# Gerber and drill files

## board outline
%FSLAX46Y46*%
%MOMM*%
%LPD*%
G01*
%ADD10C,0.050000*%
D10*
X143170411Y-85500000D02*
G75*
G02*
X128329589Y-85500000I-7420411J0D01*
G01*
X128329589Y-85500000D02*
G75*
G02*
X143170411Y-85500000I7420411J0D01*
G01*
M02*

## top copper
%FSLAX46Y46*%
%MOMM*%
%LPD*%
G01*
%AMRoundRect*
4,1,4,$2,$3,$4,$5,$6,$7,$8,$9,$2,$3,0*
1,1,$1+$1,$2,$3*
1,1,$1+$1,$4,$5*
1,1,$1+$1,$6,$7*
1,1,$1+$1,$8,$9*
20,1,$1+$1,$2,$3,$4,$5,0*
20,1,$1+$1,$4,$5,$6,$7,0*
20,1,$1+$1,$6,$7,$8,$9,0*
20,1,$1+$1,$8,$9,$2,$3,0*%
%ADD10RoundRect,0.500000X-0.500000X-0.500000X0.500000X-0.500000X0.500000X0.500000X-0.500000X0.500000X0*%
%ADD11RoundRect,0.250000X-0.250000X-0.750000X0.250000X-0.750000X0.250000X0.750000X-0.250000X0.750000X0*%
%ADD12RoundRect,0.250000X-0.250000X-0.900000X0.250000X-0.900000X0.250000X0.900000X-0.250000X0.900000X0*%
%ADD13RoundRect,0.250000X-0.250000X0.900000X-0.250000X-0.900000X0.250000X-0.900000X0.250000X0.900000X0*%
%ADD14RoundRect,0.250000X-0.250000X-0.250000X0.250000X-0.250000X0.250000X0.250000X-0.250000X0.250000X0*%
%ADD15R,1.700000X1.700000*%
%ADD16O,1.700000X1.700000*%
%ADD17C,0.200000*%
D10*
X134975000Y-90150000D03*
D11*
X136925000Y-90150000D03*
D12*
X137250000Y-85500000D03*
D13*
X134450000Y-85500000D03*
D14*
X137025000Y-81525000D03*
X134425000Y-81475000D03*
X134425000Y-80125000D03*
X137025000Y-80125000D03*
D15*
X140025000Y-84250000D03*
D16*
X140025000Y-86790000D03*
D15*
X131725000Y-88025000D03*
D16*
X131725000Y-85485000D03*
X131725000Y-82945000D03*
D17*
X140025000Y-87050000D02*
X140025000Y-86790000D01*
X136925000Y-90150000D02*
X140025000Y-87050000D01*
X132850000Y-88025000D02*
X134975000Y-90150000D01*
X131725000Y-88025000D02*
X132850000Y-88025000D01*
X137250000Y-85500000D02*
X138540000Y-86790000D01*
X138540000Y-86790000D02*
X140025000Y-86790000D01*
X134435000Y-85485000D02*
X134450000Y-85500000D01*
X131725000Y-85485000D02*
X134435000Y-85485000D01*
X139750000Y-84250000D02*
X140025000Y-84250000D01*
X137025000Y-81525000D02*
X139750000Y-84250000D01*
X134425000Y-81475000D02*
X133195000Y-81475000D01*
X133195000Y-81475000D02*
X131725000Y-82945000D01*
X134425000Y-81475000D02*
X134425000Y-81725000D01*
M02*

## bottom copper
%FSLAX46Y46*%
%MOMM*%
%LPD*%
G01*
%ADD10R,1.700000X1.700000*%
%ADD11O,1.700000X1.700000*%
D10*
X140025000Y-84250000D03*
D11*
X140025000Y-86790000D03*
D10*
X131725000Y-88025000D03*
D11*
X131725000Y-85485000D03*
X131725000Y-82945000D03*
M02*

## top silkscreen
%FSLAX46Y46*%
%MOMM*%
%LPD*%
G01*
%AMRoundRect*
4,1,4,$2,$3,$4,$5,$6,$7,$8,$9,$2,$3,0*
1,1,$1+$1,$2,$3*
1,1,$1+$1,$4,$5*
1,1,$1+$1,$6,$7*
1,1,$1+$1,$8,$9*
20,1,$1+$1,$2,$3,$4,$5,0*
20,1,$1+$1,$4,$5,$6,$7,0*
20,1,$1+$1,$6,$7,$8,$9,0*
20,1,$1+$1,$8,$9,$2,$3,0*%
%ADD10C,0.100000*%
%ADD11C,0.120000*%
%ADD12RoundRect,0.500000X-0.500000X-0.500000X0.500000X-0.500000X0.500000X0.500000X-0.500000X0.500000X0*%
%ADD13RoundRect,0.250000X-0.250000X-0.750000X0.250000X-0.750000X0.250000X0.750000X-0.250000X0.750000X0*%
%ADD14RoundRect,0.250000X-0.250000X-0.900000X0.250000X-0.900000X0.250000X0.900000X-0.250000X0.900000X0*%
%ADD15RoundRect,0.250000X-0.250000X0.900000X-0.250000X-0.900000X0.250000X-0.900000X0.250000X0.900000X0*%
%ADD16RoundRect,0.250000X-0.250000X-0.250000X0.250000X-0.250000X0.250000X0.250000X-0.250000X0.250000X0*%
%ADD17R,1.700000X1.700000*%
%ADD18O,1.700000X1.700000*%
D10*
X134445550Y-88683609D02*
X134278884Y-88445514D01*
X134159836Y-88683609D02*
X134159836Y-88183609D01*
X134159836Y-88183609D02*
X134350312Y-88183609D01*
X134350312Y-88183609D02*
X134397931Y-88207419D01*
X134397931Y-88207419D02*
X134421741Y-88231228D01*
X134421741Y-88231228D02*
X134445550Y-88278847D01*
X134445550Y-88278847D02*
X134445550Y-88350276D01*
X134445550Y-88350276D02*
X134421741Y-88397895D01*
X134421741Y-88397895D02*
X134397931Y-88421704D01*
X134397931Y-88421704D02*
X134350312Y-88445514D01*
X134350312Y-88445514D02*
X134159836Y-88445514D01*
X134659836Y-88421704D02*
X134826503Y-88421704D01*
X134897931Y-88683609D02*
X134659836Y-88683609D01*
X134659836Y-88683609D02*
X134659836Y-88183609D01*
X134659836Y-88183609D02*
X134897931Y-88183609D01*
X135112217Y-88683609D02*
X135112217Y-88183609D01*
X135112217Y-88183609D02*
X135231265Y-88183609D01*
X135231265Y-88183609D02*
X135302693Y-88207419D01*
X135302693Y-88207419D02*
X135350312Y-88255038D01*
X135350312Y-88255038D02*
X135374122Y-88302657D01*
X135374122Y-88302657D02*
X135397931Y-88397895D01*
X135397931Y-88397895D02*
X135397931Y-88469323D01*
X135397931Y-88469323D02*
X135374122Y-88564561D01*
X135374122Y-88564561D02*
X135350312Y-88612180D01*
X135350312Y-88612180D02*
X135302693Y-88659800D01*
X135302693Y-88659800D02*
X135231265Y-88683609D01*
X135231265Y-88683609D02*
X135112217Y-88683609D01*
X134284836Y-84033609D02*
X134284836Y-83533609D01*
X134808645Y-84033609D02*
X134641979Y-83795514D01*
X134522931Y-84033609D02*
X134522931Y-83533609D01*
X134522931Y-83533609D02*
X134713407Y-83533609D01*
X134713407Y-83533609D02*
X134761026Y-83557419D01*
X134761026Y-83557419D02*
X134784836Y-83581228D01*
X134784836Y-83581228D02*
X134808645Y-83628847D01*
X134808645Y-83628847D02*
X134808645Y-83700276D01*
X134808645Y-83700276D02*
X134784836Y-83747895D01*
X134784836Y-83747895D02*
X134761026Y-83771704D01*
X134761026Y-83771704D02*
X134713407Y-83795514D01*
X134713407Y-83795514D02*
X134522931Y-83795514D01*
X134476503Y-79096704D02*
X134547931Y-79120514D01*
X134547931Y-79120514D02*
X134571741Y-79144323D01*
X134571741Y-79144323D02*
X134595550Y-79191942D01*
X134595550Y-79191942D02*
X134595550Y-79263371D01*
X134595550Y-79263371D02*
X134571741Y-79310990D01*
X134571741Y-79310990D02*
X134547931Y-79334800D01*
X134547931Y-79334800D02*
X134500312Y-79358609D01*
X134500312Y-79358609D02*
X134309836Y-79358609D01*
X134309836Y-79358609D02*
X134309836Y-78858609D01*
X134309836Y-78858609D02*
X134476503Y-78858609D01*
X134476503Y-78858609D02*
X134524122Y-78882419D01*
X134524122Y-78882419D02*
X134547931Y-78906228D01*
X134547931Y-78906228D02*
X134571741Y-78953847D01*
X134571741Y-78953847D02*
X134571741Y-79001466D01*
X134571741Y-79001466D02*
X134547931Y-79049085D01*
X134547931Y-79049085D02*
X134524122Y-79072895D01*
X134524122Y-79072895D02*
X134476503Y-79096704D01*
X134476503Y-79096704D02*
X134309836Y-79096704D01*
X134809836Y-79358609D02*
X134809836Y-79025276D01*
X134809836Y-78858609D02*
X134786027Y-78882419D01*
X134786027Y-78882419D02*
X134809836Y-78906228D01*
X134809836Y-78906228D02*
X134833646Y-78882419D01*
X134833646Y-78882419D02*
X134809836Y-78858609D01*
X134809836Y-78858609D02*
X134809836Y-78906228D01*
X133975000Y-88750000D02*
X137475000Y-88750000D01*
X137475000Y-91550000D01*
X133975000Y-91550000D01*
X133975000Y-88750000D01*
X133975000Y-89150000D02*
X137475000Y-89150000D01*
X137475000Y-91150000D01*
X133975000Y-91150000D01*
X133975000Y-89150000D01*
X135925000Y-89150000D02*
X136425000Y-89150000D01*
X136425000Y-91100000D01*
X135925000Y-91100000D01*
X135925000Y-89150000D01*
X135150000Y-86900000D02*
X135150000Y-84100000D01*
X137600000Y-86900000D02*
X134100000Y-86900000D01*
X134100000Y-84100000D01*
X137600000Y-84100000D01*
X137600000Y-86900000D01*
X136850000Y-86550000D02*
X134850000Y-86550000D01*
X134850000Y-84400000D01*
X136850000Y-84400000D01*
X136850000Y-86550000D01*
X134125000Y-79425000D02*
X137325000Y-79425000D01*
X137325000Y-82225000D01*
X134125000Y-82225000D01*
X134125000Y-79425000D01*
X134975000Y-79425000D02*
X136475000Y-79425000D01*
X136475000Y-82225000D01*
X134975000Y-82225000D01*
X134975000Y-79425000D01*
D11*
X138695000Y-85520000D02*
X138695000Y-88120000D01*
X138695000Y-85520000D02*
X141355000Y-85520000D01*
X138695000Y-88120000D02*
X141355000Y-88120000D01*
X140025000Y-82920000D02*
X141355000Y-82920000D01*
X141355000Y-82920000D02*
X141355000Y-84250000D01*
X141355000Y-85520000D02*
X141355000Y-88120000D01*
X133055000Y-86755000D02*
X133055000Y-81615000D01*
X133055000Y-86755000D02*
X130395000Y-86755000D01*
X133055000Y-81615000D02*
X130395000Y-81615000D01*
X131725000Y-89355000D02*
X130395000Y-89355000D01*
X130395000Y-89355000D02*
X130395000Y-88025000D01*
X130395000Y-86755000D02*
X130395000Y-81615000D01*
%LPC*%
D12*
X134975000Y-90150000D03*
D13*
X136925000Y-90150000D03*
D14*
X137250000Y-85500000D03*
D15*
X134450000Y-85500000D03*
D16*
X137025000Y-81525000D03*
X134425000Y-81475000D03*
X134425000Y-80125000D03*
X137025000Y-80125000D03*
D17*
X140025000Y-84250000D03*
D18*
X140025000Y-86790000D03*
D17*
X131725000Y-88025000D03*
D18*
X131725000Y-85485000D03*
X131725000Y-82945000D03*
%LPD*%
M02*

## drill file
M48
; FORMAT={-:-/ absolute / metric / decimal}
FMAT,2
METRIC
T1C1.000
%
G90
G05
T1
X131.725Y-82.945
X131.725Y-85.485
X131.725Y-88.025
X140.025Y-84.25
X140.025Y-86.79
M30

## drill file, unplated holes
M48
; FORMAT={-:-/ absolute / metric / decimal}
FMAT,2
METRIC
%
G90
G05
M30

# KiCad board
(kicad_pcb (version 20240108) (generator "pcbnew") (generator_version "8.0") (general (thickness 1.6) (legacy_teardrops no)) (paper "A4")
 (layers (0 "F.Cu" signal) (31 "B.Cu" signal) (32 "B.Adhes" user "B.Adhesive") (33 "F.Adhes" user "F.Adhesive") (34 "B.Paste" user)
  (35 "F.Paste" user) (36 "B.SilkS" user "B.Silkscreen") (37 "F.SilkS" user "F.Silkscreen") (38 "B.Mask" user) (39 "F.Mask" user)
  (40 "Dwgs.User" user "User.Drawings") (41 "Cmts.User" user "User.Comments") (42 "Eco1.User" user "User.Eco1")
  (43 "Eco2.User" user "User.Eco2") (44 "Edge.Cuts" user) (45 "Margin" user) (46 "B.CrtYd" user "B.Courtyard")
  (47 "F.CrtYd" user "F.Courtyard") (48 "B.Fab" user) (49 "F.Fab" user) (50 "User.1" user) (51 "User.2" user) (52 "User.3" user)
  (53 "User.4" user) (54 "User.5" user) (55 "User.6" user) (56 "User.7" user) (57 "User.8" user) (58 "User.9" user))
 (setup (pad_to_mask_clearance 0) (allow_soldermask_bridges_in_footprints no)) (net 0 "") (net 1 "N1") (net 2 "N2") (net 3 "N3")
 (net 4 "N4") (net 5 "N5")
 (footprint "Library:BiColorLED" (layer "F.Cu") (at 135.675 84.025)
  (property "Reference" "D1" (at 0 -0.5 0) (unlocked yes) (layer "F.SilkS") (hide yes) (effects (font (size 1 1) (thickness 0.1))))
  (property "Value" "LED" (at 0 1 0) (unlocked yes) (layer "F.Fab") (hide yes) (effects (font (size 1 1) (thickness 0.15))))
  (fp_rect (start -1.55 -4.6) (end 1.65 -1.8) (stroke (width 0.1) (type default)) (fill none) (layer "F.SilkS"))
  (fp_rect (start -0.7 -4.6) (end 0.8 -1.8) (stroke (width 0.1) (type default)) (fill none) (layer "F.SilkS"))
  (pad "1" smd roundrect (at 1.35 -2.5) (size 1 1) (layers "F.Cu" "F.Paste" "F.Mask") (roundrect_rratio 0.25) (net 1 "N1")
   (thermal_bridge_angle 45))
  (pad "2" smd roundrect (at -1.25 -2.55) (size 1 1) (layers "F.Cu" "F.Paste" "F.Mask") (roundrect_rratio 0.25) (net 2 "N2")
   (thermal_bridge_angle 45))
  (pad "3" smd roundrect (at -1.25 -3.9) (size 1 1) (layers "F.Cu" "F.Paste" "F.Mask") (roundrect_rratio 0.25) (thermal_bridge_angle 45))
  (pad "4" smd roundrect (at 1.35 -3.9) (size 1 1) (layers "F.Cu" "F.Paste" "F.Mask") (roundrect_rratio 0.25) (thermal_bridge_angle 45)))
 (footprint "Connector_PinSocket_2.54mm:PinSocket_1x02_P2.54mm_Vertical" (layer "F.Cu") (at 140.025 84.25)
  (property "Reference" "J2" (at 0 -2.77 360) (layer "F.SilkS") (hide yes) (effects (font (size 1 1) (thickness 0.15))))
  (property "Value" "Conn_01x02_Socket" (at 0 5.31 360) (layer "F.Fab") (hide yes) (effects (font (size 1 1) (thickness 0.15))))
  (fp_line (start -1.33 1.27) (end -1.33 3.87) (stroke (width 0.12) (type solid)) (layer "F.SilkS"))
  (fp_line (start -1.33 1.27) (end 1.33 1.27) (stroke (width 0.12) (type solid)) (layer "F.SilkS"))
  (fp_line (start -1.33 3.87) (end 1.33 3.87) (stroke (width 0.12) (type solid)) (layer "F.SilkS"))
  (fp_line (start 0 -1.33) (end 1.33 -1.33) (stroke (width 0.12) (type solid)) (layer "F.SilkS"))
  (fp_line (start 1.33 -1.33) (end 1.33 0) (stroke (width 0.12) (type solid)) (layer "F.SilkS"))
  (fp_line (start 1.33 1.27) (end 1.33 3.87) (stroke (width 0.12) (type solid)) (layer "F.SilkS"))
  (pad "1" thru_hole rect (at 0 0) (size 1.7 1.7) (drill 1) (layers "*.Cu" "*.Mask") (remove_unused_layers no) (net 1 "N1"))
  (pad "2" thru_hole oval (at 0 2.54) (size 1.7 1.7) (drill 1) (layers "*.Cu" "*.Mask") (remove_unused_layers no) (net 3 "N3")))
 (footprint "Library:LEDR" (layer "F.Cu") (at 135.625 94.7)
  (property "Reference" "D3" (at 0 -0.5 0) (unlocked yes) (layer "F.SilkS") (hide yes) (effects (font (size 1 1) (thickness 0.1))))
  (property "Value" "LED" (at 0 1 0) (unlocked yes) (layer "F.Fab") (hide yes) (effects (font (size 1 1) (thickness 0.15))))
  (fp_rect (start -1.65 -5.95) (end 1.85 -3.15) (stroke (width 0.1) (type default)) (fill none) (layer "F.SilkS"))
  (fp_rect (start -1.65 -5.55) (end 1.85 -3.55) (stroke (width 0.1) (type default)) (fill none) (layer "F.SilkS"))
  (fp_rect (start 0.3 -5.55) (end 0.8 -3.6) (stroke (width 0.1) (type default)) (fill none) (layer "F.SilkS"))
  (pad "1" smd roundrect (at 1.3 -4.55) (size 1 2) (layers "F.Cu" "F.Paste" "F.Mask") (roundrect_rratio 0.25) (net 3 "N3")
   (thermal_bridge_angle 45))
  (pad "2" smd roundrect (at -0.65 -4.55) (size 2 2) (layers "F.Cu" "F.Paste" "F.Mask") (roundrect_rratio 0.25) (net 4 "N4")
   (thermal_bridge_angle 45)))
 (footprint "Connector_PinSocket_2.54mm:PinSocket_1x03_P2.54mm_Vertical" (layer "F.Cu") (at 131.725 88.025 180)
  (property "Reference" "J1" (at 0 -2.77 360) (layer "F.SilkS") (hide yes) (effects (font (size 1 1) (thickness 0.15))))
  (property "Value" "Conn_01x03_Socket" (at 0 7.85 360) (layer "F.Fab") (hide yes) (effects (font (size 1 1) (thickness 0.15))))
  (fp_line (start 1.33 1.27) (end 1.33 6.41) (stroke (width 0.12) (type solid)) (layer "F.SilkS"))
  (fp_line (start 1.33 -1.33) (end 1.33 0) (stroke (width 0.12) (type solid)) (layer "F.SilkS"))
  (fp_line (start 0 -1.33) (end 1.33 -1.33) (stroke (width 0.12) (type solid)) (layer "F.SilkS"))
  (fp_line (start -1.33 6.41) (end 1.33 6.41) (stroke (width 0.12) (type solid)) (layer "F.SilkS"))
  (fp_line (start -1.33 1.27) (end 1.33 1.27) (stroke (width 0.12) (type solid)) (layer "F.SilkS"))
  (fp_line (start -1.33 1.27) (end -1.33 6.41) (stroke (width 0.12) (type solid)) (layer "F.SilkS"))
  (pad "1" thru_hole rect (at 0 0 180) (size 1.7 1.7) (drill 1) (layers "*.Cu" "*.Mask") (remove_unused_layers no) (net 4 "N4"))
  (pad "2" thru_hole oval (at 0 2.54 180) (size 1.7 1.7) (drill 1) (layers "*.Cu" "*.Mask") (remove_unused_layers no) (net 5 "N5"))
  (pad "3" thru_hole oval (at 0 5.08 180) (size 1.7 1.7) (drill 1) (layers "*.Cu" "*.Mask") (remove_unused_layers no) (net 2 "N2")))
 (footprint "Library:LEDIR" (layer "F.Cu") (at 133.75 79.65 180)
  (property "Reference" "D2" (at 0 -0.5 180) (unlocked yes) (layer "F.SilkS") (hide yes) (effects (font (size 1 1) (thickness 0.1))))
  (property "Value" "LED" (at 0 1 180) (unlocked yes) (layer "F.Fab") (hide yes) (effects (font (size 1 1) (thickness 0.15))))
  (fp_line (start -1.4 -7.25) (end -1.4 -4.45) (stroke (width 0.1) (type default)) (layer "F.SilkS"))
  (fp_rect (start -3.1 -6.9) (end -1.1 -4.75) (stroke (width 0.1) (type default)) (fill none) (layer "F.SilkS"))
  (fp_rect (start -3.85 -7.25) (end -0.35 -4.45) (stroke (width 0.1) (type default)) (fill none) (layer "F.SilkS"))
  (pad "1" smd roundrect (at -3.5 -5.85) (size 1 2.3) (layers "F.Cu" "F.Paste" "F.Mask") (roundrect_rratio 0.25) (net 3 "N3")
   (thermal_bridge_angle 45))
  (pad "2" smd roundrect (at -0.7 -5.85 270) (size 2.3 1) (layers "F.Cu" "F.Paste" "F.Mask") (roundrect_rratio 0.25) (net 5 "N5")
   (thermal_bridge_angle 45)))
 (gr_circle (center 135.75 85.5) (end 142 81.5) (stroke (width 0.05) (type default)) (fill none) (layer "Edge.Cuts"))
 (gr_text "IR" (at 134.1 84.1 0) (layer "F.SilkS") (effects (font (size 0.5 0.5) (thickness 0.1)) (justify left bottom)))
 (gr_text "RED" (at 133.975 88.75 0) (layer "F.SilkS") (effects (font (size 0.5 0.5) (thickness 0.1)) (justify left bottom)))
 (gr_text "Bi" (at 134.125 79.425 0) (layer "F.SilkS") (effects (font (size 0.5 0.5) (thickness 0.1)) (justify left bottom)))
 (segment (start 133.195 81.475) (end 131.725 82.945) (width 0.2) (layer "F.Cu") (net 2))
 (segment (start 134.425 81.475) (end 133.195 81.475) (width 0.2) (layer "F.Cu") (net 2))
 (segment (start 134.425 81.475) (end 134.425 81.725) (width 0.2) (layer "F.Cu") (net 2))
 (segment (start 137.025 81.525) (end 139.75 84.25) (width 0.2) (layer "F.Cu") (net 1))
 (segment (start 139.75 84.25) (end 140.025 84.25) (width 0.2) (layer "F.Cu") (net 1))
 (segment (start 131.725 85.485) (end 134.435 85.485) (width 0.2) (layer "F.Cu") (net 5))
 (segment (start 134.435 85.485) (end 134.45 85.5) (width 0.2) (layer "F.Cu") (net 5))
 (segment (start 140.025 87.05) (end 140.025 86.79) (width 0.2) (layer "F.Cu") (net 3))
 (segment (start 136.925 90.15) (end 140.025 87.05) (width 0.2) (layer "F.Cu") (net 3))
 (segment (start 138.54 86.79) (end 140.025 86.79) (width 0.2) (layer "F.Cu") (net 3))
 (segment (start 137.25 85.5) (end 138.54 86.79) (width 0.2) (layer "F.Cu") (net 3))
 (segment (start 132.85 88.025) (end 134.975 90.15) (width 0.2) (layer "F.Cu") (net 4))
 (segment (start 131.725 88.025) (end 132.85 88.025) (width 0.2) (layer "F.Cu") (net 4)))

